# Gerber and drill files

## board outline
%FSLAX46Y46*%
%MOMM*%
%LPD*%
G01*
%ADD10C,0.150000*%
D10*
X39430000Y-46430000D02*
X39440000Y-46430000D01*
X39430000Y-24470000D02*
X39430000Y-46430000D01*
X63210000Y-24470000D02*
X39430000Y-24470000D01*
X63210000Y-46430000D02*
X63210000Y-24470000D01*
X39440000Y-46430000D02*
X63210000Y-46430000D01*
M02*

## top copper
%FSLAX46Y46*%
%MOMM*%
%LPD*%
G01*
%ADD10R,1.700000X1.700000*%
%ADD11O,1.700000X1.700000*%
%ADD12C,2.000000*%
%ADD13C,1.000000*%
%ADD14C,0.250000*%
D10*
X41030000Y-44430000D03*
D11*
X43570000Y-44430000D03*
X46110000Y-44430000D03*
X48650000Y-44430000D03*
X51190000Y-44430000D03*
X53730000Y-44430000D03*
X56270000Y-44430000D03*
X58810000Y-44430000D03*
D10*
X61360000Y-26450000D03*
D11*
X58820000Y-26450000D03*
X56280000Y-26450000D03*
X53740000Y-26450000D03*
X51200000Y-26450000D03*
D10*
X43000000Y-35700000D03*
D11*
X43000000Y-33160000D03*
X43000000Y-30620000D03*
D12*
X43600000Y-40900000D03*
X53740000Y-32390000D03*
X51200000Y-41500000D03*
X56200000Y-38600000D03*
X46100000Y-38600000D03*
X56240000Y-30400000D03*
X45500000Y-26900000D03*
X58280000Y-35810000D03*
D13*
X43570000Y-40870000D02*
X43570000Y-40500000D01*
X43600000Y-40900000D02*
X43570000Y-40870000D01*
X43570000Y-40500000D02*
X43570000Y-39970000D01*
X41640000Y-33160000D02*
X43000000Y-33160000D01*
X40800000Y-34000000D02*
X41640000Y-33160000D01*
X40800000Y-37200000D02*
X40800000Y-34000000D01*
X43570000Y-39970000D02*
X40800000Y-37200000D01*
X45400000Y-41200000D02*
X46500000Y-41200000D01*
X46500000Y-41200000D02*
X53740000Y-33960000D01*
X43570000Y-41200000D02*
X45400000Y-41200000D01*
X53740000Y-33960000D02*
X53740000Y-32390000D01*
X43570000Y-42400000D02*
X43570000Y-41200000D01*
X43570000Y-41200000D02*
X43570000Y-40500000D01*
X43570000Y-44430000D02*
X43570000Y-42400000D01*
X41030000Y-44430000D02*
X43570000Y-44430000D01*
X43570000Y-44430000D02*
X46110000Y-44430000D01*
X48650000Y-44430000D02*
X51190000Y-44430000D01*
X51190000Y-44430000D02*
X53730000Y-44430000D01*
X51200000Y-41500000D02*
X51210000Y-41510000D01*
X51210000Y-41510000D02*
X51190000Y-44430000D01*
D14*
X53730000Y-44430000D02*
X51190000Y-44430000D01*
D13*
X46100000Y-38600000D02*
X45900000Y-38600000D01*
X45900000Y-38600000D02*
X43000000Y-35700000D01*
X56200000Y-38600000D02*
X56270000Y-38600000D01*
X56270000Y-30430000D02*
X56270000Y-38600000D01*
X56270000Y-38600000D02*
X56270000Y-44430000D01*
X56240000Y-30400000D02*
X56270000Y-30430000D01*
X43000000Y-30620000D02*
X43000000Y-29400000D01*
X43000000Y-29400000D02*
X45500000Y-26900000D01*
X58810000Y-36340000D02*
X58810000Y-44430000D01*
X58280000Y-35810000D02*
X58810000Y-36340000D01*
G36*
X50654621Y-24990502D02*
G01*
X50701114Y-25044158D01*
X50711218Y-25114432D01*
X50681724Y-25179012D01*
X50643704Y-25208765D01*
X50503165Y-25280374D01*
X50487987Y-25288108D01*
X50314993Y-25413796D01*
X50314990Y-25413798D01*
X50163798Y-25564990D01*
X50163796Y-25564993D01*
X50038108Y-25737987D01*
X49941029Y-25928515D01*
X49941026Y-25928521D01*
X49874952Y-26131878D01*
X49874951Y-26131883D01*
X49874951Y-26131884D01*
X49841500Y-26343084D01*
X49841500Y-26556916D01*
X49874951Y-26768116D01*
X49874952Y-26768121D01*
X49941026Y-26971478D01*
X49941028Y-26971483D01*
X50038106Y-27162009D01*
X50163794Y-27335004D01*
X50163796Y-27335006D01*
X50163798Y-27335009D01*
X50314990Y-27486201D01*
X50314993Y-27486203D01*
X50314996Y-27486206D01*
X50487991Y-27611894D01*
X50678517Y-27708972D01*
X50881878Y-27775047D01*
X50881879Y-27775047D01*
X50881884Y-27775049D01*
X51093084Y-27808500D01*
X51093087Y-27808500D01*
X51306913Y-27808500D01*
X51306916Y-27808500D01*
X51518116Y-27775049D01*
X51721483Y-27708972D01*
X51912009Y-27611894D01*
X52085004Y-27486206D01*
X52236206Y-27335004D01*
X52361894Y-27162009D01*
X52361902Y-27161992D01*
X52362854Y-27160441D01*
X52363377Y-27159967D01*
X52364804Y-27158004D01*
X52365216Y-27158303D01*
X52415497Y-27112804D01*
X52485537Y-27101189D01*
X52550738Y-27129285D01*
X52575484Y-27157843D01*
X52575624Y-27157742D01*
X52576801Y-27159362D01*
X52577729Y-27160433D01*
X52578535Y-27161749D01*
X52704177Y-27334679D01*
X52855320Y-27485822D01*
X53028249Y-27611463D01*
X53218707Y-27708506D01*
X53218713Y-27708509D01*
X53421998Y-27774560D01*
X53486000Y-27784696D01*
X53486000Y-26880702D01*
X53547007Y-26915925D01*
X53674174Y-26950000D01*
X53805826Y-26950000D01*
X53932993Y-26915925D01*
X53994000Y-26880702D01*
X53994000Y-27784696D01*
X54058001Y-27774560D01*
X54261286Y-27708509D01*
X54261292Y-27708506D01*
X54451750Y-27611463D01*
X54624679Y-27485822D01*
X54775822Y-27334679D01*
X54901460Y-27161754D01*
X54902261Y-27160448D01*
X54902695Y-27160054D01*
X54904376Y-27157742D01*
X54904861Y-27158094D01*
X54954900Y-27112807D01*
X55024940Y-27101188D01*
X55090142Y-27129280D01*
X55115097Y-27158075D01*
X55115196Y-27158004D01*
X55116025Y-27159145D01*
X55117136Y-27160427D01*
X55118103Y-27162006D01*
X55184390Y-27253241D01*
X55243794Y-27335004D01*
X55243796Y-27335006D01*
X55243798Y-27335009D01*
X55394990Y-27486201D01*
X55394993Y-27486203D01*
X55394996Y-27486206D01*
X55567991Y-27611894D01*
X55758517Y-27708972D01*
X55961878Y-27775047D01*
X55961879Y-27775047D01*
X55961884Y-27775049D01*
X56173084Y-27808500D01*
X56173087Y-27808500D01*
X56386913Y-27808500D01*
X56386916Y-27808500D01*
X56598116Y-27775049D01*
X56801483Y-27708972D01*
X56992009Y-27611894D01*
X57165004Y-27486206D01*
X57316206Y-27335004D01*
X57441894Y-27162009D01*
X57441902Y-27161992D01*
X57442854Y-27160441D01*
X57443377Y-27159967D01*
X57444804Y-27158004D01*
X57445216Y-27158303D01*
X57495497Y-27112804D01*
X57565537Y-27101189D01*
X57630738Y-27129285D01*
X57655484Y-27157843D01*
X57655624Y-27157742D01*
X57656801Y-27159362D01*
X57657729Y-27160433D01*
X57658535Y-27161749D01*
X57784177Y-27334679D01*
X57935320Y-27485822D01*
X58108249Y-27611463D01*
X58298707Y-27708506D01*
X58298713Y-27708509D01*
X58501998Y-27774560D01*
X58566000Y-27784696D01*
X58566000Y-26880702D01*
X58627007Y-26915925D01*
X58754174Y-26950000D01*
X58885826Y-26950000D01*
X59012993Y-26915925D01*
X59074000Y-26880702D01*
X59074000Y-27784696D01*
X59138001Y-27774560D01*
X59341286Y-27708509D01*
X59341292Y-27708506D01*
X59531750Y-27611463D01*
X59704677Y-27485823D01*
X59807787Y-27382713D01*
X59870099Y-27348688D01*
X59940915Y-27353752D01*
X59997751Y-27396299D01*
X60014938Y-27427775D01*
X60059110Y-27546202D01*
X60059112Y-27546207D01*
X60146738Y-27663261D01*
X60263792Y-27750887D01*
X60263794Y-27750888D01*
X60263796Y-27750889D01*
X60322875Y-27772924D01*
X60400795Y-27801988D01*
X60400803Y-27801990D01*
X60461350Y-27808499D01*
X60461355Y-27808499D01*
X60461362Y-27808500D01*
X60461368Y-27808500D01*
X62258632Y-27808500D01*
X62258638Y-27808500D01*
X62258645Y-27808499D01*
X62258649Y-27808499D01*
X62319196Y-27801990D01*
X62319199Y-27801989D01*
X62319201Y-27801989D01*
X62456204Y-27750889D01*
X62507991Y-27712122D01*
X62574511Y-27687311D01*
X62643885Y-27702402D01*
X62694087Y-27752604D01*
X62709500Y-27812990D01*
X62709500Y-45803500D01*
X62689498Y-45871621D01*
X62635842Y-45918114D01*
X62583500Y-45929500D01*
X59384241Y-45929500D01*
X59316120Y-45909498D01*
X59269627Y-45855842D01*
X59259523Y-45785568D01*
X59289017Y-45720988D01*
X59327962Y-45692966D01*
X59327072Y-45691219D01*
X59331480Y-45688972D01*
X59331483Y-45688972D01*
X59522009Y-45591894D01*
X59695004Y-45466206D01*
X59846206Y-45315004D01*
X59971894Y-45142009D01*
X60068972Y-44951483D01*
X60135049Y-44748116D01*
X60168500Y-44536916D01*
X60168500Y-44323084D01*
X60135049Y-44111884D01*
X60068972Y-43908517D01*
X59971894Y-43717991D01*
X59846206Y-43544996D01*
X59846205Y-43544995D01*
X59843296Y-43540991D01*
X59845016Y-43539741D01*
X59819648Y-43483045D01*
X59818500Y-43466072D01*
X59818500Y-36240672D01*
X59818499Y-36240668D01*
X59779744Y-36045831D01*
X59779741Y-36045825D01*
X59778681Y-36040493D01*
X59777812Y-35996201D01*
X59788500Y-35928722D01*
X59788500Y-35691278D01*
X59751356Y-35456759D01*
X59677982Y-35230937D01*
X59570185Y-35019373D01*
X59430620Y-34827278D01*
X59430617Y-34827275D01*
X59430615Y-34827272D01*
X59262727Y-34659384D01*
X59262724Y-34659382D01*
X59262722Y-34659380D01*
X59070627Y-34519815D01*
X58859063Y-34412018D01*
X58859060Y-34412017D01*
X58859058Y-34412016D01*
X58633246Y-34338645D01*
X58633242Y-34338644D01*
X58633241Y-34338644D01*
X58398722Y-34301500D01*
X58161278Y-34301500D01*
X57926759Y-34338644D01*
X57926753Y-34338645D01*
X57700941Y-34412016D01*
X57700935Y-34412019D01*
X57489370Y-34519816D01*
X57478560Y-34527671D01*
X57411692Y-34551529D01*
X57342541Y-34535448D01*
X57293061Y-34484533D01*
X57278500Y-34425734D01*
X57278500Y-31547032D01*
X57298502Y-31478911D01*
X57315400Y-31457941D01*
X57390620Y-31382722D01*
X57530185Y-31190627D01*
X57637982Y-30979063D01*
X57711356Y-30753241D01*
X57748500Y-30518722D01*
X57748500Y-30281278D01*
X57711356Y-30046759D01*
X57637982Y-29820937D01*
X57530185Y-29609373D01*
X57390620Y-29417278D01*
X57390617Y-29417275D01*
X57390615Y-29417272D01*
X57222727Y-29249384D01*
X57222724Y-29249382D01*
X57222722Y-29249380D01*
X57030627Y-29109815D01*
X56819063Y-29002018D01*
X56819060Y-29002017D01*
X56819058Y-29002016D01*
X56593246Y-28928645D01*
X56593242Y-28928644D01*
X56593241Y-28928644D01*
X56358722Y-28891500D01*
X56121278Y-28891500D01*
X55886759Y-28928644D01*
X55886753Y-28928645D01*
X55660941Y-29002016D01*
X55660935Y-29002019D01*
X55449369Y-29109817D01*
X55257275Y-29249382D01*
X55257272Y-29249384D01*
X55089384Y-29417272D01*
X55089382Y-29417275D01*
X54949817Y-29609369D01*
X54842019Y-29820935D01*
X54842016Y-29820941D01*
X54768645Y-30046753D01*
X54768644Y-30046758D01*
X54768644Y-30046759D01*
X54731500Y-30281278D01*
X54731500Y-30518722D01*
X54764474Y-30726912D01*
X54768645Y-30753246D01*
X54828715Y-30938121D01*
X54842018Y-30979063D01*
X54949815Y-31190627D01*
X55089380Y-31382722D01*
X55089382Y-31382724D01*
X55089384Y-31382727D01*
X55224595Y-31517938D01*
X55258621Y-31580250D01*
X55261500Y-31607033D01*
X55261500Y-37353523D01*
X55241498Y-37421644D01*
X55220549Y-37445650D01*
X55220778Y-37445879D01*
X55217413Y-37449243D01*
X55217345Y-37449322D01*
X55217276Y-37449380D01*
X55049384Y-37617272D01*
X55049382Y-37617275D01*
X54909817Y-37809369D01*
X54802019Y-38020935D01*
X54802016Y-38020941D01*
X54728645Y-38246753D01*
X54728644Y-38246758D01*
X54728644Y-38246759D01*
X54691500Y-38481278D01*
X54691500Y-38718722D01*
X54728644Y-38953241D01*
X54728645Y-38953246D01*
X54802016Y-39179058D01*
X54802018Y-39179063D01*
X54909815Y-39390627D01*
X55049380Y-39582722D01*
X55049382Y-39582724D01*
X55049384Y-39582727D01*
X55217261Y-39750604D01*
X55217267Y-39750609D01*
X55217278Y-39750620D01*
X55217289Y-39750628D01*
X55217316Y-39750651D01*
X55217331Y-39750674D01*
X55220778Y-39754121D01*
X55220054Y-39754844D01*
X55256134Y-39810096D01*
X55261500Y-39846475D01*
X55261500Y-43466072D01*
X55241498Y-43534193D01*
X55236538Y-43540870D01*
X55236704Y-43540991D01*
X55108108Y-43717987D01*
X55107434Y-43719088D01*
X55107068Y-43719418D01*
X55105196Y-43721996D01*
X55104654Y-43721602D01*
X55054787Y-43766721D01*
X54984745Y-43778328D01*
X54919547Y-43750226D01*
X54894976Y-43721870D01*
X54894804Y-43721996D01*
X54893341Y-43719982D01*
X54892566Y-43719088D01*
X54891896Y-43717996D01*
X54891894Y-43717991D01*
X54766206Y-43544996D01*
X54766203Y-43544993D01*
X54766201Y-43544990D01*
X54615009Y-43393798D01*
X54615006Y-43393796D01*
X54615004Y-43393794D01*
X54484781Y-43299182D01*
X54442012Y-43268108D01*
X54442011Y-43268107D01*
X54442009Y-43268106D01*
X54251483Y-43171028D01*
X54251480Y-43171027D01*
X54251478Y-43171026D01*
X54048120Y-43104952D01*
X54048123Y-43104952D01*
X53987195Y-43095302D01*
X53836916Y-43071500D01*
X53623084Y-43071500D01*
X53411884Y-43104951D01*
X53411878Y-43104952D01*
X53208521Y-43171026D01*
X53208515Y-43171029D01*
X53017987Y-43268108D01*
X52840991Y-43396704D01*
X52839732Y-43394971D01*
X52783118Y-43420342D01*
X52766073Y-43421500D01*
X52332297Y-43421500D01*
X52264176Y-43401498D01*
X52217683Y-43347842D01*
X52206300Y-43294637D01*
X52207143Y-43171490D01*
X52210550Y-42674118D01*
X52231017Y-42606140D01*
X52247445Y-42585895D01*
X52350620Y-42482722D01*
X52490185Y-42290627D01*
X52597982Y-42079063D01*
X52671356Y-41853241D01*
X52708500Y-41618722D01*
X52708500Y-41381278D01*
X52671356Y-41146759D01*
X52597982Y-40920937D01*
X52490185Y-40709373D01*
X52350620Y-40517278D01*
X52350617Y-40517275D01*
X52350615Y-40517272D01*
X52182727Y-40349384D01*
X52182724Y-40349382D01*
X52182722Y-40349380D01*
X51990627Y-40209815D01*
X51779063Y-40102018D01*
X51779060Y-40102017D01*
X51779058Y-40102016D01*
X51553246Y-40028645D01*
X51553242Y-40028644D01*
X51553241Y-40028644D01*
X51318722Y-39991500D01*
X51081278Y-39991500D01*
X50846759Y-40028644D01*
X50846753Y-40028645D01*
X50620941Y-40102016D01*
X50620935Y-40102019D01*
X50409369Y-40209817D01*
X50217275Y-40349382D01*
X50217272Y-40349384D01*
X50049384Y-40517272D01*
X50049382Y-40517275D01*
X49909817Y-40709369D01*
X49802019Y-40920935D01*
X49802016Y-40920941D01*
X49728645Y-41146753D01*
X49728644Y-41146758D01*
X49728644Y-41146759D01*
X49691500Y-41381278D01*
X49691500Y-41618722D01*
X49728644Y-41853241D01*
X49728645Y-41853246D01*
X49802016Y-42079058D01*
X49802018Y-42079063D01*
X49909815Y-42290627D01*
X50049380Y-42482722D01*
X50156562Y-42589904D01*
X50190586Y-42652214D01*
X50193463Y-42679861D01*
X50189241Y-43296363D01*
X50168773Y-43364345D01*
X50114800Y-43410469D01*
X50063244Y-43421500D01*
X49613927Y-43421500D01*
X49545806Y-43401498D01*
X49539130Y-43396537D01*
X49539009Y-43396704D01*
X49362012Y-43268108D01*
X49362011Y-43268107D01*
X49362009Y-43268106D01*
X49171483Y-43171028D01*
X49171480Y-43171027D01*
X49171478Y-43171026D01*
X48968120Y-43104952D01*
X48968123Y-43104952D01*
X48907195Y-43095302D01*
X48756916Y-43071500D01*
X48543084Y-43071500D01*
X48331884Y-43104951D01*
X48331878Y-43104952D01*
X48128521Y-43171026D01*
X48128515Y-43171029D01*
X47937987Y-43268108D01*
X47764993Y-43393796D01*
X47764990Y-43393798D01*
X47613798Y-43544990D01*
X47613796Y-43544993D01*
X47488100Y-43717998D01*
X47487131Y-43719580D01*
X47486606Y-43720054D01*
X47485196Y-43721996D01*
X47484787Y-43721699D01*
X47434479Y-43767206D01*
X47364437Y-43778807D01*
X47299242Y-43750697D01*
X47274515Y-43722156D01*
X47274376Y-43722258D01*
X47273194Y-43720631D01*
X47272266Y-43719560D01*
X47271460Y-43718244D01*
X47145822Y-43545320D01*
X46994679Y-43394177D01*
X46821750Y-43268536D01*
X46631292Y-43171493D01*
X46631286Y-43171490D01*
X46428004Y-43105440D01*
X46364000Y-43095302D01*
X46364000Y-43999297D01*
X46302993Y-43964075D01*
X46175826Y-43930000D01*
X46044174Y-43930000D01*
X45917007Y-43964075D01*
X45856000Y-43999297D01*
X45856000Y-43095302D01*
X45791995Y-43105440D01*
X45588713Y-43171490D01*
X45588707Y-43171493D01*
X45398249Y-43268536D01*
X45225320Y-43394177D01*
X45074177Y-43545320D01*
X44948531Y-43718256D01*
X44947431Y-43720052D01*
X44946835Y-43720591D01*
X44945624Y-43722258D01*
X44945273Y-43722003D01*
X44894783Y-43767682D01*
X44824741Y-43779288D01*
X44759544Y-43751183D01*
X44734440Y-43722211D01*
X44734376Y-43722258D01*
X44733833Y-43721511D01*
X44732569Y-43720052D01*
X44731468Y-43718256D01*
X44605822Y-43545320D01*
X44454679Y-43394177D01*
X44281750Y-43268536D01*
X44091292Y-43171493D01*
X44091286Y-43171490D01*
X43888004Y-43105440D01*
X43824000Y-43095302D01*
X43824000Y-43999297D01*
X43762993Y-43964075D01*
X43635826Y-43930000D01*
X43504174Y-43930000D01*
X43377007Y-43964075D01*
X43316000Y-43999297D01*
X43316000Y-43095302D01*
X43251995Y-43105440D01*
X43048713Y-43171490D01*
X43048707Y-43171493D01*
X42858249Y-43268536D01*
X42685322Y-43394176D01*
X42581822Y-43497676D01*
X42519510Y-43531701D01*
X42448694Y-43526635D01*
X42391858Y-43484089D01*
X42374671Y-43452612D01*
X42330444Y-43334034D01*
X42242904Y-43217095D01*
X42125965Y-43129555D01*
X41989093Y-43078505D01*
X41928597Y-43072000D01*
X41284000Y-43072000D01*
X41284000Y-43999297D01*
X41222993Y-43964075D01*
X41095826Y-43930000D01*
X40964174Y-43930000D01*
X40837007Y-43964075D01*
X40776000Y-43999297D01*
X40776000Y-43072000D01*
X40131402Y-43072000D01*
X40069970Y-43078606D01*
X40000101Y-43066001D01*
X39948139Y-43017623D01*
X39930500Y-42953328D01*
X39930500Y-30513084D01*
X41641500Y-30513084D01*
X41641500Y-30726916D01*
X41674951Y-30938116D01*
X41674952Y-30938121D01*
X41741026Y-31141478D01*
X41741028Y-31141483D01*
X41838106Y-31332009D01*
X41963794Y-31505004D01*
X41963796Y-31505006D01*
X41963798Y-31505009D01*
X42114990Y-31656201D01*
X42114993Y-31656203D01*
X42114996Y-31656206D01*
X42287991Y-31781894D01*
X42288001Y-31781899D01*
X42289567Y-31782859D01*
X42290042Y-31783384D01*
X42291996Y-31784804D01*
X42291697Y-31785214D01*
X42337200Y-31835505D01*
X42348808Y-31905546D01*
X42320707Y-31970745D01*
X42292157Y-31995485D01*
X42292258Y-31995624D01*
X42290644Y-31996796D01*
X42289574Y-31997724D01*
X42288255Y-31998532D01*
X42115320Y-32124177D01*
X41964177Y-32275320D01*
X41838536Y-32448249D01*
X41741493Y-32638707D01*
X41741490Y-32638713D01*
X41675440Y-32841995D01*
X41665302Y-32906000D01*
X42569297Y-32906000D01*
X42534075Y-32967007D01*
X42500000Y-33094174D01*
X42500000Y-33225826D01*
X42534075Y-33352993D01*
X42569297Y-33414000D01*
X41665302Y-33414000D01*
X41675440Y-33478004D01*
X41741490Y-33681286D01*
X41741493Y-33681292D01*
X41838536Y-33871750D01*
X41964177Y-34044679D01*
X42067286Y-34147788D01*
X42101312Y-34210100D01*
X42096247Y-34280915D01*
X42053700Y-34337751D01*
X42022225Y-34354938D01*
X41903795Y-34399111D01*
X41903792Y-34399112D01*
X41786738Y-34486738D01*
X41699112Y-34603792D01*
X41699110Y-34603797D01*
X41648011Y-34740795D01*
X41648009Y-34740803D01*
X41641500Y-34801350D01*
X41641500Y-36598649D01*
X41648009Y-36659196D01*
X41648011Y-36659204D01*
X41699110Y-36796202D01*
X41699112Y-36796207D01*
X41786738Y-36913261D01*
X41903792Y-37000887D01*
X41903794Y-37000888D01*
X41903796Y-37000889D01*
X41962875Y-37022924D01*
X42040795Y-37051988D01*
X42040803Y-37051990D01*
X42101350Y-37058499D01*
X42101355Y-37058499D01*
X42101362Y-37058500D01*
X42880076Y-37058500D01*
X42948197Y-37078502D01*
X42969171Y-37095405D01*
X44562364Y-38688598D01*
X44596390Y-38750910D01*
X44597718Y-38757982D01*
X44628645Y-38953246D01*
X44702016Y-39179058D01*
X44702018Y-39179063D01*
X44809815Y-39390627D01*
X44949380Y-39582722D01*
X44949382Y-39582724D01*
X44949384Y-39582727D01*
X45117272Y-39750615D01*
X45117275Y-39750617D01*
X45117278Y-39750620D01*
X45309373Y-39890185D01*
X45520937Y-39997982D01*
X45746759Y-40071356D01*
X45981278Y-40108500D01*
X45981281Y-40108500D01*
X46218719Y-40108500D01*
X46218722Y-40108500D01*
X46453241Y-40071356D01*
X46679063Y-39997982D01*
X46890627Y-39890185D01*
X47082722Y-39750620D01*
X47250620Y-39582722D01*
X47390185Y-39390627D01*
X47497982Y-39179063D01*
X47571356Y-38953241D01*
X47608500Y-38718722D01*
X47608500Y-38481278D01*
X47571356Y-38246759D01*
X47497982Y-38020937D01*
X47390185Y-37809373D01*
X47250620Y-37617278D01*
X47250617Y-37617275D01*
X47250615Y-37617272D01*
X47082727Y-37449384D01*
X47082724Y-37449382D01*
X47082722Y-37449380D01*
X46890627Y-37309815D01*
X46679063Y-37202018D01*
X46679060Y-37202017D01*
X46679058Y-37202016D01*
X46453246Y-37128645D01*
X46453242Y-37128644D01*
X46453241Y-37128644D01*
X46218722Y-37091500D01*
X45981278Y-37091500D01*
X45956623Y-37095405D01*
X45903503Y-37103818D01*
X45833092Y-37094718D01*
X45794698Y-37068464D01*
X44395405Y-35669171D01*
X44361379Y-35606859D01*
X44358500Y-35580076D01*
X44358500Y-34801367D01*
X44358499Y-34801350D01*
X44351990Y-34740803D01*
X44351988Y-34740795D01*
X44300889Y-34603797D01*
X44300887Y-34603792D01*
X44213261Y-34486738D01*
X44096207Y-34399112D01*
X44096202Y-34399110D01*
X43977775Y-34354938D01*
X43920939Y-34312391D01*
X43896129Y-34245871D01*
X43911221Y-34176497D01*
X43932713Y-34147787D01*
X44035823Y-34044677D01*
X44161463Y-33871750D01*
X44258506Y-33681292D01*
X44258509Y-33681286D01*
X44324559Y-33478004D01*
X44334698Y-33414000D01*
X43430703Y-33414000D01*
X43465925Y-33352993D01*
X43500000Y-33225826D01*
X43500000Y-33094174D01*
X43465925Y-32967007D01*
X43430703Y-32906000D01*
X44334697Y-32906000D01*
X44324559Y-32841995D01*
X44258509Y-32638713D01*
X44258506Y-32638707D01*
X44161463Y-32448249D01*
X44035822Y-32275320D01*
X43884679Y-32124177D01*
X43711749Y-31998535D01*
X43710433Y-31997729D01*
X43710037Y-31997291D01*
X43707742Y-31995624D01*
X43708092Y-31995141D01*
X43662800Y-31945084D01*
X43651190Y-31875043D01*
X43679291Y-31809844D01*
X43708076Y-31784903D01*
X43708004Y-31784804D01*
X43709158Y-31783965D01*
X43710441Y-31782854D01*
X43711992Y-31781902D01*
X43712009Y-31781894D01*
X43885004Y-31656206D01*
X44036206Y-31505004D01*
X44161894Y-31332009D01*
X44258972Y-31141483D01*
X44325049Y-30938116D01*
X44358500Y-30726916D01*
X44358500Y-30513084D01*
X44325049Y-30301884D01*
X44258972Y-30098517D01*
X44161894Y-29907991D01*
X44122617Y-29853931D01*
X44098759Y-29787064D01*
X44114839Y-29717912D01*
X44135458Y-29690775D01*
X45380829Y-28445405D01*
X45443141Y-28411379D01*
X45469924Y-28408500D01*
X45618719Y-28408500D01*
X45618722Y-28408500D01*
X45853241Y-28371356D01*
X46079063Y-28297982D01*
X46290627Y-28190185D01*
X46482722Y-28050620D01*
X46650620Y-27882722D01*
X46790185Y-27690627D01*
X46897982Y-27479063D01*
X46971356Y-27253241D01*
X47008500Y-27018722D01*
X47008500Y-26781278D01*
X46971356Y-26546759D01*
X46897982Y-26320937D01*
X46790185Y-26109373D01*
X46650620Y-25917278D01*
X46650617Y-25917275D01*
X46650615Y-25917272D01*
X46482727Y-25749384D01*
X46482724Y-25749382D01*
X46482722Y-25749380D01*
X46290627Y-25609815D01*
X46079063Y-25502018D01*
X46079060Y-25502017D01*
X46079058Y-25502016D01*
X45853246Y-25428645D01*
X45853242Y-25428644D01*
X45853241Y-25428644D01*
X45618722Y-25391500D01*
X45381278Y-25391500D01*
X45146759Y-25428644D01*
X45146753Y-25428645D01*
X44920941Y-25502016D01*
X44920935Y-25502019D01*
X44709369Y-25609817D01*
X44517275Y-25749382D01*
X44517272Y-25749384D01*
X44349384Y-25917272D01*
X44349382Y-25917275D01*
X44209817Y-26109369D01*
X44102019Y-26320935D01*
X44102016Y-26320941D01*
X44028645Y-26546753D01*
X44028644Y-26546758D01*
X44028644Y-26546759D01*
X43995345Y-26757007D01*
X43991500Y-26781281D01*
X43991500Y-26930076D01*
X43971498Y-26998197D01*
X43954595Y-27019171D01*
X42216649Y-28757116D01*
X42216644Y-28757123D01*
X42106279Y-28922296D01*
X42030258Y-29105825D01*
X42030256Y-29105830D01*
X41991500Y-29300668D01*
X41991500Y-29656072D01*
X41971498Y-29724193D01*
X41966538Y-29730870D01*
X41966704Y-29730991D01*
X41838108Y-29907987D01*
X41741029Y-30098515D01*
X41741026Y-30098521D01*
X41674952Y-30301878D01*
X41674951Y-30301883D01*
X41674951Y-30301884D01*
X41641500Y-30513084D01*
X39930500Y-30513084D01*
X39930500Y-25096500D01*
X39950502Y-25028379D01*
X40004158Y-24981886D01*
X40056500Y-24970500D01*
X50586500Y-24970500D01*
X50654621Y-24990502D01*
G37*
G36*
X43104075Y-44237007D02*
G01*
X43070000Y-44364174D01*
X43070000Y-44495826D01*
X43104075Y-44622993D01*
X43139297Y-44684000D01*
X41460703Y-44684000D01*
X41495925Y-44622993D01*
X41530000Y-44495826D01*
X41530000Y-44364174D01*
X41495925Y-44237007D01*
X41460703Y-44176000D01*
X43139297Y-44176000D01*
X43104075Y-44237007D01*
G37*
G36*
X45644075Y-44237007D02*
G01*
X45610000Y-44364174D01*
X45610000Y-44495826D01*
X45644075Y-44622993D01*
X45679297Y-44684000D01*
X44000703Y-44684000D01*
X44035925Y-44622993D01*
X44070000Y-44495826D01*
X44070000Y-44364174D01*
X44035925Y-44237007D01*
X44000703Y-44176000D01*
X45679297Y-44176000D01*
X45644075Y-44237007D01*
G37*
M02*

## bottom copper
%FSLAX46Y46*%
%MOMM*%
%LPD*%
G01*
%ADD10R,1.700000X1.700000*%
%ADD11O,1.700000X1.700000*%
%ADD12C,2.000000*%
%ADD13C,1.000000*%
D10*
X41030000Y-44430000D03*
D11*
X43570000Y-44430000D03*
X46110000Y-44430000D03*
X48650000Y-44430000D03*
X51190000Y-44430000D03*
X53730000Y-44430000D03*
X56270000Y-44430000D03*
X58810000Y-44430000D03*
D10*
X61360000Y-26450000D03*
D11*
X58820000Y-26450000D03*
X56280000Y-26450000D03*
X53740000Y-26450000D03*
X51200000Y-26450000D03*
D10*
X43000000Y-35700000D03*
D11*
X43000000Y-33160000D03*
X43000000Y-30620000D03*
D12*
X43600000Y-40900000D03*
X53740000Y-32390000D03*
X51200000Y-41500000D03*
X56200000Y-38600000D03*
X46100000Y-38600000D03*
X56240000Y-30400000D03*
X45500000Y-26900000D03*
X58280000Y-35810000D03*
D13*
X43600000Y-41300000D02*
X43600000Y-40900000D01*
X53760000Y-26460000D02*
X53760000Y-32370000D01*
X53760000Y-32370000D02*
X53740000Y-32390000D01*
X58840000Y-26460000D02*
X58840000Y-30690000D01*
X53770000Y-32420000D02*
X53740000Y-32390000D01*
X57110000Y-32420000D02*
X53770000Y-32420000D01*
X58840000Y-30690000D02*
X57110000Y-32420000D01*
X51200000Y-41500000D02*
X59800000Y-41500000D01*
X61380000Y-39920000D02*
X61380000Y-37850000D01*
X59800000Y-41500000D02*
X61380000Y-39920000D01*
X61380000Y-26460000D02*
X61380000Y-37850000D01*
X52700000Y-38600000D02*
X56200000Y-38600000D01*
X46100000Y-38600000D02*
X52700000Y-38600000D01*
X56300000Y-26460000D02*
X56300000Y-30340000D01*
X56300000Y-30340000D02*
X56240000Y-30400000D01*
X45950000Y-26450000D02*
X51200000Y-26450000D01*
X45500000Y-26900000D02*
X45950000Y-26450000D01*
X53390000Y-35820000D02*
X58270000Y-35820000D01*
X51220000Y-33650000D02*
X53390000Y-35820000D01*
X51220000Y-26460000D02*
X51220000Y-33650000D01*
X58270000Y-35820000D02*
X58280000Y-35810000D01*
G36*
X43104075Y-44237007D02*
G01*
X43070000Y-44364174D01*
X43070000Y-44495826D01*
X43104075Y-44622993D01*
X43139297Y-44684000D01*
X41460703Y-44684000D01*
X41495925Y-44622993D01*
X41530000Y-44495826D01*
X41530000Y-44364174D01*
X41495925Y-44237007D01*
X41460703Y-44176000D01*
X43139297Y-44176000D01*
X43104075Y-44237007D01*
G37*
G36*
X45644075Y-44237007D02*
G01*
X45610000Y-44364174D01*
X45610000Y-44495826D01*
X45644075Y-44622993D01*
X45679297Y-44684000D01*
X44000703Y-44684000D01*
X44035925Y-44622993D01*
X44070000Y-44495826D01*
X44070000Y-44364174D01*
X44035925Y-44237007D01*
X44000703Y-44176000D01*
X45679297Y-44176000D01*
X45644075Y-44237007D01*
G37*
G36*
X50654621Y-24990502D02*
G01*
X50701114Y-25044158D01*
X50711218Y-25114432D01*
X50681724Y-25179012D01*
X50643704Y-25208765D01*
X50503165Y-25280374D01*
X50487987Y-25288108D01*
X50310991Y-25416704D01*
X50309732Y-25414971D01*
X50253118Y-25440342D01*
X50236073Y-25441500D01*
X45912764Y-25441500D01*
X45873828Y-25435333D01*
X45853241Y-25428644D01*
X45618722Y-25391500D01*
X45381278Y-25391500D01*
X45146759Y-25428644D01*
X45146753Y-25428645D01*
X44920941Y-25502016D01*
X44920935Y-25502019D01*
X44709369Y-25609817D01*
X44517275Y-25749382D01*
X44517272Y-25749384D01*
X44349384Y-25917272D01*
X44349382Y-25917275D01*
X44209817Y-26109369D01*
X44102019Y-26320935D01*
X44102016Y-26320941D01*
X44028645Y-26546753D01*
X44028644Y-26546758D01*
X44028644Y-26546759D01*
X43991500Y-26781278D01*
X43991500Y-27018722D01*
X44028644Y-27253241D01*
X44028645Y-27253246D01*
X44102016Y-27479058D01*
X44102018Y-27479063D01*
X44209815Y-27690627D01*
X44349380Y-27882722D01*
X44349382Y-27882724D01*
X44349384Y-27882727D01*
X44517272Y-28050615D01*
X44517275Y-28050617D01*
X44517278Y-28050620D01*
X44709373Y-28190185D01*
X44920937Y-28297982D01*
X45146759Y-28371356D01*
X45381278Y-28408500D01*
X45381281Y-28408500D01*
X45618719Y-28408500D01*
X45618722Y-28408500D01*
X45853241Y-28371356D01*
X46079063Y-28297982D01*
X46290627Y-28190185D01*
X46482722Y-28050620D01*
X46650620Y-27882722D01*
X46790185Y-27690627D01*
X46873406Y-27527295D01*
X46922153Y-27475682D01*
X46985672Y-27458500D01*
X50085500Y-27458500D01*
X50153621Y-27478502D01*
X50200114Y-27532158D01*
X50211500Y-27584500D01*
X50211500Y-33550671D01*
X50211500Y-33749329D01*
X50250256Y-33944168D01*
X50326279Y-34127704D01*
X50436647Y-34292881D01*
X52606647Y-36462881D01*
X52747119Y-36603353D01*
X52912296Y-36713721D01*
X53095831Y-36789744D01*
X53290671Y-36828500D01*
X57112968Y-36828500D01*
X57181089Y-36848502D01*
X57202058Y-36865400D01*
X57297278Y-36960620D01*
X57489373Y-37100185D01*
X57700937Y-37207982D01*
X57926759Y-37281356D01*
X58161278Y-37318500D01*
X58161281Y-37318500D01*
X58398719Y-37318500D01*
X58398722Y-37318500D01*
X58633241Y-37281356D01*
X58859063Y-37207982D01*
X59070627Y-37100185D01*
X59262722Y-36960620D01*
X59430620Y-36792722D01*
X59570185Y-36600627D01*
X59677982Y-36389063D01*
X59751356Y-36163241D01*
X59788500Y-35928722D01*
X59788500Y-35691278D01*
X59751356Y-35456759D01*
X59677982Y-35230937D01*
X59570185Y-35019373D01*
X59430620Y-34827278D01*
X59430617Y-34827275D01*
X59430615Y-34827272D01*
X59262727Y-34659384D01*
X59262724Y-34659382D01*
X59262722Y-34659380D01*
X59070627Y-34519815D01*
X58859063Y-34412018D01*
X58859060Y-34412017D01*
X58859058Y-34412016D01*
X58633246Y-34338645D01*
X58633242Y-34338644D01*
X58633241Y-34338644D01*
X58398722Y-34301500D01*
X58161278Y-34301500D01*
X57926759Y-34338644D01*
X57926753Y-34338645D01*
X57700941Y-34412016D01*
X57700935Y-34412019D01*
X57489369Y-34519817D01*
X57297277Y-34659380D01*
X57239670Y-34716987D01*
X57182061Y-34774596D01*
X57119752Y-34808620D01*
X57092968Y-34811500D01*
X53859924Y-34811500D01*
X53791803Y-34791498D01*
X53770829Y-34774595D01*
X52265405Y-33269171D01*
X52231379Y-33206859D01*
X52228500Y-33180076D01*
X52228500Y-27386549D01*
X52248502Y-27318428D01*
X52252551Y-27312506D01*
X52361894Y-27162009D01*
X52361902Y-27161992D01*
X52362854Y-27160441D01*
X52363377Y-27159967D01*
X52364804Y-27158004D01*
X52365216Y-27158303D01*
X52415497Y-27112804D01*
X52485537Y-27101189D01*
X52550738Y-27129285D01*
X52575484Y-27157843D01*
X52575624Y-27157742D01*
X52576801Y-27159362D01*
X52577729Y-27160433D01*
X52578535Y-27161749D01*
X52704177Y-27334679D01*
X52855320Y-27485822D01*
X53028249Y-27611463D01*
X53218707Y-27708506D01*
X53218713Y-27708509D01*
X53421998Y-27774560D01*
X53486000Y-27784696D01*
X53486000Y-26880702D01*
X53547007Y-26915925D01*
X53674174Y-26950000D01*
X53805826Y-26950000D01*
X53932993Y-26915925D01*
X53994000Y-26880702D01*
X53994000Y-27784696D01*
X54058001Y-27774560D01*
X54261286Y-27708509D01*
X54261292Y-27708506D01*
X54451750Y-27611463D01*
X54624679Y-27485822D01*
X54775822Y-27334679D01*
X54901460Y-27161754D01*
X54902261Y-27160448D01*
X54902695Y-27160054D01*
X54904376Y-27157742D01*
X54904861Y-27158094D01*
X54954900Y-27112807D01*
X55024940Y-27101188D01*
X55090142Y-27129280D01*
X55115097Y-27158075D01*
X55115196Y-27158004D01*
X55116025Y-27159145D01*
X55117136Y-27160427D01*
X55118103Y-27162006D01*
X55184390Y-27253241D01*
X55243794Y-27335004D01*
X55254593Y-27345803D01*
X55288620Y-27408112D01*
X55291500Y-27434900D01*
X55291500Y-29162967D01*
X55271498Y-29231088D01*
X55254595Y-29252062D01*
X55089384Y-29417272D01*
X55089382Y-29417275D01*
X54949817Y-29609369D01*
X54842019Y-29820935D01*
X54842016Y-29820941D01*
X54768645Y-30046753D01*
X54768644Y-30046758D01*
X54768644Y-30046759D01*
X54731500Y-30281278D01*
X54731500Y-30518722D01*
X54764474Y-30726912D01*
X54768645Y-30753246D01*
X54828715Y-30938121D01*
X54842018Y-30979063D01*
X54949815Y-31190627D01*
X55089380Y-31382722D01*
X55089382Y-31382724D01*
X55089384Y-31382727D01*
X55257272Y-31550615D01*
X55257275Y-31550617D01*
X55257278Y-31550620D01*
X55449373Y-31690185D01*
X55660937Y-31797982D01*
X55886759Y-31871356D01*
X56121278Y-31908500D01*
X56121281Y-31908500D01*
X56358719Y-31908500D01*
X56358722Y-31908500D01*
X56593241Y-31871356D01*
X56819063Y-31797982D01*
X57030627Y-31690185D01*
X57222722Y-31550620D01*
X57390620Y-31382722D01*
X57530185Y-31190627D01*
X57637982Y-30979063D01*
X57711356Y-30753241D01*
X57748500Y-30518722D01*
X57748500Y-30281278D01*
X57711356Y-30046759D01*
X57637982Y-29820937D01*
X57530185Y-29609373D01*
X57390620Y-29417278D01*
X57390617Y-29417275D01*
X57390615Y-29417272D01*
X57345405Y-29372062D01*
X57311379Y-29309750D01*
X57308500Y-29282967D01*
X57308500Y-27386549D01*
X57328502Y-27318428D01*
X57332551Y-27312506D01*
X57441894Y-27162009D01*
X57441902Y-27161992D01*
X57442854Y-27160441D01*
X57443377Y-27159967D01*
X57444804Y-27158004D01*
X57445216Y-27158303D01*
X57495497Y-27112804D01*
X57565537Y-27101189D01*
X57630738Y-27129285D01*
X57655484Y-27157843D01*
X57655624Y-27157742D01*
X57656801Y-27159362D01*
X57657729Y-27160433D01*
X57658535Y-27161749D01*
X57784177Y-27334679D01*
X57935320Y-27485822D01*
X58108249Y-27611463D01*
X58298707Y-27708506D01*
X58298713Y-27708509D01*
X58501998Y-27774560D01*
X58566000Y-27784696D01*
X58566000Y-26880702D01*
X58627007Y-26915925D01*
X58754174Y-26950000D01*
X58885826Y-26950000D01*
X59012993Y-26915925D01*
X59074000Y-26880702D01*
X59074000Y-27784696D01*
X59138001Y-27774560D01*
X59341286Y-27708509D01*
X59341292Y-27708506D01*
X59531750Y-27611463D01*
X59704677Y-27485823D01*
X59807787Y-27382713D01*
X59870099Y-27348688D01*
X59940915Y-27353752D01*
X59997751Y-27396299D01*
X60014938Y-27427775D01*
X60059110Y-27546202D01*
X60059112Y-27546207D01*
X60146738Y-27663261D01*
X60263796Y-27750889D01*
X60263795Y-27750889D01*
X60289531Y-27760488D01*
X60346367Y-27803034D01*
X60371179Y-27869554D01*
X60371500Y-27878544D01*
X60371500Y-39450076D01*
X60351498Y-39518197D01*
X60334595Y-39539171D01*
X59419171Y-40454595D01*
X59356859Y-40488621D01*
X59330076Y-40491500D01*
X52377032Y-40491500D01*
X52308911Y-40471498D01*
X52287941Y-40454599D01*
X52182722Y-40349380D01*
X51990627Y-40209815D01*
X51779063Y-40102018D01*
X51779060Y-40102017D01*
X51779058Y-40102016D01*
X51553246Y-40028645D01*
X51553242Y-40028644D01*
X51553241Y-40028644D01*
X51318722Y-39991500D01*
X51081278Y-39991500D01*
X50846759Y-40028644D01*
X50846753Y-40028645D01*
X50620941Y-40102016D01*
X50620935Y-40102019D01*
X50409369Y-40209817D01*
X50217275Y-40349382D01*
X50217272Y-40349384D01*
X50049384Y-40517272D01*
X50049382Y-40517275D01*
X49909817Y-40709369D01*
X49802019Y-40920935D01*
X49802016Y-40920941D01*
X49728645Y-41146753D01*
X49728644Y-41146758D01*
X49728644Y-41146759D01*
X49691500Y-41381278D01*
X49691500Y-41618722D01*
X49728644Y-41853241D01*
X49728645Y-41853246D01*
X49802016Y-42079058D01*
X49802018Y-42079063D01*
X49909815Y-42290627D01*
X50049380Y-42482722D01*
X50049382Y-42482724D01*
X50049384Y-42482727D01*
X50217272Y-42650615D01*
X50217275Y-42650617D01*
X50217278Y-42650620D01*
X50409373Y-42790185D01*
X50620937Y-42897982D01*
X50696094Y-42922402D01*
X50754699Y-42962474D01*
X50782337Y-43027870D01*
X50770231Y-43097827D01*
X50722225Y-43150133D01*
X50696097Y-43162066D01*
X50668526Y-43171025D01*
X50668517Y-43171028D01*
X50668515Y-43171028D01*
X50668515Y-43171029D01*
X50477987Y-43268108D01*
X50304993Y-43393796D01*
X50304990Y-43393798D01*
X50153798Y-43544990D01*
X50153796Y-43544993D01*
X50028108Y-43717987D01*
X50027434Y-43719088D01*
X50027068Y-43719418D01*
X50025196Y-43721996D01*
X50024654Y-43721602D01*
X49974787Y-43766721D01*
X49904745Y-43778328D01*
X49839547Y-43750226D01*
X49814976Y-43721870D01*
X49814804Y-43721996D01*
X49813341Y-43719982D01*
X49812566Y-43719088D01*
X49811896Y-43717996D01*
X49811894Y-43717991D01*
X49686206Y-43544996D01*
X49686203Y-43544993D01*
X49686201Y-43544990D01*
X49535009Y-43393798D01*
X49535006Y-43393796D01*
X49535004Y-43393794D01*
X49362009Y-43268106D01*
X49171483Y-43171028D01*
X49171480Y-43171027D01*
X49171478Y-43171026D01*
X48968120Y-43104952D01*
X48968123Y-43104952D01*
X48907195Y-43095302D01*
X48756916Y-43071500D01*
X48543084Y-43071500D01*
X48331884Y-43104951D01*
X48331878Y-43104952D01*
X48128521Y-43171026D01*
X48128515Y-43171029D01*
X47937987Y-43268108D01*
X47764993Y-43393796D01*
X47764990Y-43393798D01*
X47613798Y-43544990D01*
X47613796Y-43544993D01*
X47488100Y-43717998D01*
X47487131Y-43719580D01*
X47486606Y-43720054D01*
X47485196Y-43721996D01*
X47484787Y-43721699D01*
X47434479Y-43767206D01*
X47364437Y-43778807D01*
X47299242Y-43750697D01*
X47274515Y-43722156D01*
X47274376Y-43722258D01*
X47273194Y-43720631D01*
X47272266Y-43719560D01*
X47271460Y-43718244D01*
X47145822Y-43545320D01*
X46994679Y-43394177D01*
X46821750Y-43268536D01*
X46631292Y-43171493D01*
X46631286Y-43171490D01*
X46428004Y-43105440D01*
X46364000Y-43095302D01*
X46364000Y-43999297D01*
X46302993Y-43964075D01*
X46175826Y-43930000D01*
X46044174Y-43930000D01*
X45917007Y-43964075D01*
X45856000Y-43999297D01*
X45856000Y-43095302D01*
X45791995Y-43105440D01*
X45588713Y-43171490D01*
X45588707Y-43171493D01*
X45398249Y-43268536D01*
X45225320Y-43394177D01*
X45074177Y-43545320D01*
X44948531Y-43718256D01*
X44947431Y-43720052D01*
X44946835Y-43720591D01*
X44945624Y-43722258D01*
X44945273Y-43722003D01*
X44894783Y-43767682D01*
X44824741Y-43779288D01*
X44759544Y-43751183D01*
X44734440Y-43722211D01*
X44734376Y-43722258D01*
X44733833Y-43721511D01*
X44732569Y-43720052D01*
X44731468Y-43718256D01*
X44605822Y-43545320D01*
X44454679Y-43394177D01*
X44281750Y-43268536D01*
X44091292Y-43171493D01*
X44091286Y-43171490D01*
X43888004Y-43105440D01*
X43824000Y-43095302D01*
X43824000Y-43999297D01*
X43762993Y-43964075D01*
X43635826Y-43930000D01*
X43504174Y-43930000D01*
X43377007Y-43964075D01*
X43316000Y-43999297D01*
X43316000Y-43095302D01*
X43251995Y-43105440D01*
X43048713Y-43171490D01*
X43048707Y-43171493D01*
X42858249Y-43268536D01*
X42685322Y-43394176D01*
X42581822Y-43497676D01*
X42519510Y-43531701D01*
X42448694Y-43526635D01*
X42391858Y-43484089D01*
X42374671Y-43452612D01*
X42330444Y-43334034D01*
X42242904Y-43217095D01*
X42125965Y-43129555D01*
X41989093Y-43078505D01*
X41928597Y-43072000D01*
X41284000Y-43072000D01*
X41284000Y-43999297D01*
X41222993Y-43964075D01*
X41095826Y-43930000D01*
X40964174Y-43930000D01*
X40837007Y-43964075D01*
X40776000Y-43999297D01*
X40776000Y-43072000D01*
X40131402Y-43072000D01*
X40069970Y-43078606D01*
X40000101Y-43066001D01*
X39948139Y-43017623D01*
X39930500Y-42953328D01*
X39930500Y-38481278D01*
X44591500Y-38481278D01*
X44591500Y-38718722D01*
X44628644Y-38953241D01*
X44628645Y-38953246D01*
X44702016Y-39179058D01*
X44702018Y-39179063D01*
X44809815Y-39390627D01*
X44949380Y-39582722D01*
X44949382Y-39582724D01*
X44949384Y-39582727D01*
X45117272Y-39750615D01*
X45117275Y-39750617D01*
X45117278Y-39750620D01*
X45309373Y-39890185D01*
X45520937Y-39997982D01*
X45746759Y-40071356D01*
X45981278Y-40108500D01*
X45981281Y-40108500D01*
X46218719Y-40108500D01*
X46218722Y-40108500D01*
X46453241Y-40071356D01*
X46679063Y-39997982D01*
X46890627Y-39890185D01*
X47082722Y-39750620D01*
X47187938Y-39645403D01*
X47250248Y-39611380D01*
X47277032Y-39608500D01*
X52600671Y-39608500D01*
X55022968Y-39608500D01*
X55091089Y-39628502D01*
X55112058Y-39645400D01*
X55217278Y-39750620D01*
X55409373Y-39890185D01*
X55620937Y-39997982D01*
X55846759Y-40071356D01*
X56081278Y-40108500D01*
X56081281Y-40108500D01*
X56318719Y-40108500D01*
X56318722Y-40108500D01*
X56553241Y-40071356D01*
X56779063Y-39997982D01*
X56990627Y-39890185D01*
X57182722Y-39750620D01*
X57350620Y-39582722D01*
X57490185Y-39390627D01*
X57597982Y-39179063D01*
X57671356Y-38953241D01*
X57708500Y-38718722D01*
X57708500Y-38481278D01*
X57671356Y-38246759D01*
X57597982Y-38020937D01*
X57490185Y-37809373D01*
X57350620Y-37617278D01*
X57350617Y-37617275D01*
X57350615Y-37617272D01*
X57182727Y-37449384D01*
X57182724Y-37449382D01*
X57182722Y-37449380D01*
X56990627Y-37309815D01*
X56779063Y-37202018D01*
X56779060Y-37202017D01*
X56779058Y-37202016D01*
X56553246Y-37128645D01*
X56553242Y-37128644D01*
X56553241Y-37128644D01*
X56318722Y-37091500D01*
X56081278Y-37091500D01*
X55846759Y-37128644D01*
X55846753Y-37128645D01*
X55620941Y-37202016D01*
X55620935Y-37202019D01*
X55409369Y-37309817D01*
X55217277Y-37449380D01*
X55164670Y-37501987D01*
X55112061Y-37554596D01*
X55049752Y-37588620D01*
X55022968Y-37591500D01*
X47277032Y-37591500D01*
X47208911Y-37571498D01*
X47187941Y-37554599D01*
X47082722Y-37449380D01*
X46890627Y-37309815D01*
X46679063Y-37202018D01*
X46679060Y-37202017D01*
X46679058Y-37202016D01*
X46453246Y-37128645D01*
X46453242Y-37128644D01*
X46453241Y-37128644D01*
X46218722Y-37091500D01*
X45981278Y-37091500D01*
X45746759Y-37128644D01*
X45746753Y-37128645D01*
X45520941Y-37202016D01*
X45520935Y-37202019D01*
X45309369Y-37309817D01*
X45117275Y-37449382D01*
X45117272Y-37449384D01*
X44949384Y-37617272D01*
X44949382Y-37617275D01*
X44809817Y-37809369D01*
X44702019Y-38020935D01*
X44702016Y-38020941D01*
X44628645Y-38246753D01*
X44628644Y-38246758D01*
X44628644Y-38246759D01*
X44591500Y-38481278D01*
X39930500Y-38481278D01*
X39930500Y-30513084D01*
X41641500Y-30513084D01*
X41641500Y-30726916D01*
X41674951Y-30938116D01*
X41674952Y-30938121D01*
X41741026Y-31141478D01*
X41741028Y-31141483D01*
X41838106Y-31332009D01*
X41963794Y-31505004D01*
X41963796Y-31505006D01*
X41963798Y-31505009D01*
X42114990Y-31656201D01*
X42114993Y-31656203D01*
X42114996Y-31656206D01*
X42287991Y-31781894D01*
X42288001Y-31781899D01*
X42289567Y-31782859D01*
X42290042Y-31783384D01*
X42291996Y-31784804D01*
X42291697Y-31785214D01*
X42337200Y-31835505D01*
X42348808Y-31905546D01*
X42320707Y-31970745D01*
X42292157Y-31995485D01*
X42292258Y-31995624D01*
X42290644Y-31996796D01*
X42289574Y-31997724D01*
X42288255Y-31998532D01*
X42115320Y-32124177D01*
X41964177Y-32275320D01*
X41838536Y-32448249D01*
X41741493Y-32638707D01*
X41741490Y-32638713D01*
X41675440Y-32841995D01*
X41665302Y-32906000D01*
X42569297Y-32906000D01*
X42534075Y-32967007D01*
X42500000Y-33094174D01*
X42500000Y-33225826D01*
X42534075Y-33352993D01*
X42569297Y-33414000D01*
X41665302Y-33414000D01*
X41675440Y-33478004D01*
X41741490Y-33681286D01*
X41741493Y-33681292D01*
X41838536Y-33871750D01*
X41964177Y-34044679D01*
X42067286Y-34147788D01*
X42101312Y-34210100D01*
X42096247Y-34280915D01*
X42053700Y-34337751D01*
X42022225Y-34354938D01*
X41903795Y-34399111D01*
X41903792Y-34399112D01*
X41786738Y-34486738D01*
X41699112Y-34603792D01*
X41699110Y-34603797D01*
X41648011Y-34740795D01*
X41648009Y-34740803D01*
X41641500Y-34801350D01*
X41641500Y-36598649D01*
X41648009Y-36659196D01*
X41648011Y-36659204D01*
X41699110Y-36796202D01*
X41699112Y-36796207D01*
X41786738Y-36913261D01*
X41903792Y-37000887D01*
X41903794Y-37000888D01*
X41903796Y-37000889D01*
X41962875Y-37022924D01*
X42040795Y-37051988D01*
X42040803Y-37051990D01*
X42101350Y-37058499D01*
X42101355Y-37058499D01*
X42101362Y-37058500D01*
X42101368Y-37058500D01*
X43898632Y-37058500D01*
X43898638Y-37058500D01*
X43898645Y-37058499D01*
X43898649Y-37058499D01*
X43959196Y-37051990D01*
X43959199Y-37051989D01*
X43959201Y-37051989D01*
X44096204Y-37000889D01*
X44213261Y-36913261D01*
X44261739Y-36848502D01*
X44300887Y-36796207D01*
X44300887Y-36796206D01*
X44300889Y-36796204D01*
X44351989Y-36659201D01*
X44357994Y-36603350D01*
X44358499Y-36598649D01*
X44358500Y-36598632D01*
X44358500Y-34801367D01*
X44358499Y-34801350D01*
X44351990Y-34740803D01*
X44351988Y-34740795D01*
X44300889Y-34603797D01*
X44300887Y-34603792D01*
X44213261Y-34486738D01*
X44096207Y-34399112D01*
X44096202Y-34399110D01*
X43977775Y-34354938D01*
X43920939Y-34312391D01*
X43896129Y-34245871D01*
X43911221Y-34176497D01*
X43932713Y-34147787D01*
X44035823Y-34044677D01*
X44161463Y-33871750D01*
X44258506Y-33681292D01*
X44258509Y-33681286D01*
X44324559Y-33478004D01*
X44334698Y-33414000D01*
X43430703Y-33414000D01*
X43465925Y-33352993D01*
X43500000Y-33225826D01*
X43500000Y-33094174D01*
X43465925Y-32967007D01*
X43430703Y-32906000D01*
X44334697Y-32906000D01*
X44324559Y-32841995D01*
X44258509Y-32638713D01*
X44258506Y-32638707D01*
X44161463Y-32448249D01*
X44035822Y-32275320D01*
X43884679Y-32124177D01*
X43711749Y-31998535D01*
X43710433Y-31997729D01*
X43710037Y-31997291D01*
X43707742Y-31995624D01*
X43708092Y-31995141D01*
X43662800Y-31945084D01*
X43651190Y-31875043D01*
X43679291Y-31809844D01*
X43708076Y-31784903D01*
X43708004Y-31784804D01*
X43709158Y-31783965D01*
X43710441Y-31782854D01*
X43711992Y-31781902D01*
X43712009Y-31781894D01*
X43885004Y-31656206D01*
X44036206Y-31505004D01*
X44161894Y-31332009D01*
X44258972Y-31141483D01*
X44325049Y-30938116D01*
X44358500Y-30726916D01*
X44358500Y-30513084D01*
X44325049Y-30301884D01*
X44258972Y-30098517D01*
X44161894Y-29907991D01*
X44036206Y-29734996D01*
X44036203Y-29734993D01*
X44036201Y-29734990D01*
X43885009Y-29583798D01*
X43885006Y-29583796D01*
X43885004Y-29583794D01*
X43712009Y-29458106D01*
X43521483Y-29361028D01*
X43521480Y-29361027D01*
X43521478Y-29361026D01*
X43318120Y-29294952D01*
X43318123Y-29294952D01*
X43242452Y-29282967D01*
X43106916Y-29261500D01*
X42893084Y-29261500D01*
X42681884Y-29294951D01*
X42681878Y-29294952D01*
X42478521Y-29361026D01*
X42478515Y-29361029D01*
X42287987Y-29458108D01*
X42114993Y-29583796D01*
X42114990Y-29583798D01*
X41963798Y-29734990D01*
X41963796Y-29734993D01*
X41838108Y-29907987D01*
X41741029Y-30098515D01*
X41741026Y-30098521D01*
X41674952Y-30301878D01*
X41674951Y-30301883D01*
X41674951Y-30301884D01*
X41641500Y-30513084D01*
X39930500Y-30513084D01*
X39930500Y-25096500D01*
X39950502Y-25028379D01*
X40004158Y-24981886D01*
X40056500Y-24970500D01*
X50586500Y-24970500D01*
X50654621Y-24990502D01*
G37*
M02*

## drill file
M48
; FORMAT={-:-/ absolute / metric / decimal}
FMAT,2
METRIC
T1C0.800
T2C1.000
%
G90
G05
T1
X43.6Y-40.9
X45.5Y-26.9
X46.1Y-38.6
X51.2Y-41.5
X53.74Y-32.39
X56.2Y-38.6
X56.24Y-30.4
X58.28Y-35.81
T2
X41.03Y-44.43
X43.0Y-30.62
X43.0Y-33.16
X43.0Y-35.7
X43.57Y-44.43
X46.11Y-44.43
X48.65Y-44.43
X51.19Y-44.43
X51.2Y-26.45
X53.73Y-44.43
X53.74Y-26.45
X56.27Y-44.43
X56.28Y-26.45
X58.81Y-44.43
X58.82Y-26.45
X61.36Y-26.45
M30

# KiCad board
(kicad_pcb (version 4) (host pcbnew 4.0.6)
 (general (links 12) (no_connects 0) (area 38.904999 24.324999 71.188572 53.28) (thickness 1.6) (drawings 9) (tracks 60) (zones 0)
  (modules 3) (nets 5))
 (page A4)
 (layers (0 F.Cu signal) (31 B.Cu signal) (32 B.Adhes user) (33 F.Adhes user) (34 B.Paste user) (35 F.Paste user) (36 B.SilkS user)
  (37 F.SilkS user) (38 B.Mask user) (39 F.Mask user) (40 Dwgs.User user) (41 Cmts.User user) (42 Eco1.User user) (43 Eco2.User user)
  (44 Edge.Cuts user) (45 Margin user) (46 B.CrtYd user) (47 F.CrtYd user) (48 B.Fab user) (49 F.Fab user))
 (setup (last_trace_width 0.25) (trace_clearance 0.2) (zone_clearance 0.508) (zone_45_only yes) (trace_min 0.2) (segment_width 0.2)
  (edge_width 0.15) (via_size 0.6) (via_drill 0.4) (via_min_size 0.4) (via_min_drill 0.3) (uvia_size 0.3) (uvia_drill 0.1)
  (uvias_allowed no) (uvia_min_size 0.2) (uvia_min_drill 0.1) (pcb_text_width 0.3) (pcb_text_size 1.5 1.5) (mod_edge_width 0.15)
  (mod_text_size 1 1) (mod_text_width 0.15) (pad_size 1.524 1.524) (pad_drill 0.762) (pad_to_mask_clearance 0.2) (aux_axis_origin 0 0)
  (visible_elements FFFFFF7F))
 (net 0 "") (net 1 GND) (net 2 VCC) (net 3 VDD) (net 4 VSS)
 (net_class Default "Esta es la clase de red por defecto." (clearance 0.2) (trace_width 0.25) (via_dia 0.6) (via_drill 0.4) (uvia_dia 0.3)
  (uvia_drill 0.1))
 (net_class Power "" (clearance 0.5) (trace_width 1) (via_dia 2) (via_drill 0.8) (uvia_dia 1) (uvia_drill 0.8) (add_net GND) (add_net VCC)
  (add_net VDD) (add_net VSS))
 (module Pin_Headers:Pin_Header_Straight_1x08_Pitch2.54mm (layer B.Cu) (at 41.03 44.43 270)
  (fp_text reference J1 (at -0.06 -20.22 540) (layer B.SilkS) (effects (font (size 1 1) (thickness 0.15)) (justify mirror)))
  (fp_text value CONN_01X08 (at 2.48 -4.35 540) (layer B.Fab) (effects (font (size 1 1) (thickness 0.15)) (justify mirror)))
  (pad 1 thru_hole rect (at 0 0 270) (size 1.7 1.7) (drill 1) (layers *.Cu *.Mask) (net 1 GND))
  (pad 2 thru_hole oval (at 0 -2.54 270) (size 1.7 1.7) (drill 1) (layers *.Cu *.Mask) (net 1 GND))
  (pad 3 thru_hole oval (at 0 -5.08 270) (size 1.7 1.7) (drill 1) (layers *.Cu *.Mask) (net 1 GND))
  (pad 4 thru_hole oval (at 0 -7.62 270) (size 1.7 1.7) (drill 1) (layers *.Cu *.Mask) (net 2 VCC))
  (pad 5 thru_hole oval (at 0 -10.16 270) (size 1.7 1.7) (drill 1) (layers *.Cu *.Mask) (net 2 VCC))
  (pad 6 thru_hole oval (at 0 -12.7 270) (size 1.7 1.7) (drill 1) (layers *.Cu *.Mask) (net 2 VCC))
  (pad 7 thru_hole oval (at 0 -15.24 270) (size 1.7 1.7) (drill 1) (layers *.Cu *.Mask) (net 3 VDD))
  (pad 8 thru_hole oval (at 0 -17.78 270) (size 1.7 1.7) (drill 1) (layers *.Cu *.Mask) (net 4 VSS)))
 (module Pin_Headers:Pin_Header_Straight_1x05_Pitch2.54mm (layer F.Cu) (at 61.36 26.45 270)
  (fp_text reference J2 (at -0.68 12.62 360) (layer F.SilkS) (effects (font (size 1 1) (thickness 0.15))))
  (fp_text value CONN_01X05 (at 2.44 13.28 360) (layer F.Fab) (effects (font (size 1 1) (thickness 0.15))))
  (pad 1 thru_hole rect (at 0 0 270) (size 1.7 1.7) (drill 1) (layers *.Cu *.Mask) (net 2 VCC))
  (pad 2 thru_hole oval (at 0 2.54 270) (size 1.7 1.7) (drill 1) (layers *.Cu *.Mask) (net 1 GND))
  (pad 3 thru_hole oval (at 0 5.08 270) (size 1.7 1.7) (drill 1) (layers *.Cu *.Mask) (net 3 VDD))
  (pad 4 thru_hole oval (at 0 7.62 270) (size 1.7 1.7) (drill 1) (layers *.Cu *.Mask) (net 1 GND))
  (pad 5 thru_hole oval (at 0 10.16 270) (size 1.7 1.7) (drill 1) (layers *.Cu *.Mask) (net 4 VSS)))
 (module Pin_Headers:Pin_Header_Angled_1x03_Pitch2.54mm (layer B.Cu) (at 43 35.7)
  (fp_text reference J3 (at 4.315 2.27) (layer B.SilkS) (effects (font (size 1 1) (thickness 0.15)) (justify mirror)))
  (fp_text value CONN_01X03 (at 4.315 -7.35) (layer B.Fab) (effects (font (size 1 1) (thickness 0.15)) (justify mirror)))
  (pad 1 thru_hole rect (at 0 0) (size 1.7 1.7) (drill 1) (layers *.Cu *.Mask) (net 3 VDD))
  (pad 2 thru_hole oval (at 0 -2.54) (size 1.7 1.7) (drill 1) (layers *.Cu *.Mask) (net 1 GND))
  (pad 3 thru_hole oval (at 0 -5.08) (size 1.7 1.7) (drill 1) (layers *.Cu *.Mask) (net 4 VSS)))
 (gr_line (start 39.43 46.43) (end 39.44 46.43) (angle 90) (layer Edge.Cuts) (width 0.15))
 (gr_line (start 39.43 24.47) (end 39.43 46.43) (angle 90) (layer Edge.Cuts) (width 0.15))
 (gr_line (start 63.21 24.47) (end 39.43 24.47) (angle 90) (layer Edge.Cuts) (width 0.15))
 (gr_line (start 63.21 46.43) (end 63.21 24.47) (angle 90) (layer Edge.Cuts) (width 0.15))
 (gr_line (start 39.44 46.43) (end 63.21 46.43) (angle 90) (layer Edge.Cuts) (width 0.15))
 (segment (start 43.6 41.3) (end 43.6 40.9) (width 1) (layer B.Cu) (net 1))
 (segment (start 43.57 40.87) (end 43.57 40.5) (width 1) (layer F.Cu) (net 1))
 (segment (start 43.6 40.9) (end 43.57 40.87) (width 1) (layer F.Cu) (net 1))
 (via (at 43.6 40.9) (size 2) (drill 0.8) (layers F.Cu B.Cu) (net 1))
 (segment (start 43.57 40.5) (end 43.57 39.97) (width 1) (layer F.Cu) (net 1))
 (segment (start 41.64 33.16) (end 43 33.16) (width 1) (layer F.Cu) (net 1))
 (segment (start 40.8 34) (end 41.64 33.16) (width 1) (layer F.Cu) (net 1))
 (segment (start 40.8 37.2) (end 40.8 34) (width 1) (layer F.Cu) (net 1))
 (segment (start 43.57 39.97) (end 40.8 37.2) (width 1) (layer F.Cu) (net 1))
 (segment (start 45.4 41.2) (end 46.5 41.2) (width 1) (layer F.Cu) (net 1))
 (segment (start 46.5 41.2) (end 53.74 33.96) (width 1) (layer F.Cu) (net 1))
 (segment (start 43.57 41.2) (end 45.4 41.2) (width 1) (layer F.Cu) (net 1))
 (via (at 53.74 32.39) (size 2) (drill 0.8) (layers F.Cu B.Cu) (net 1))
 (segment (start 53.74 33.96) (end 53.74 32.39) (width 1) (layer F.Cu) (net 1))
 (segment (start 43.57 42.4) (end 43.57 41.2) (width 1) (layer F.Cu) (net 1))
 (segment (start 43.57 41.2) (end 43.57 40.5) (width 1) (layer F.Cu) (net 1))
 (segment (start 43.57 44.43) (end 43.57 42.4) (width 1) (layer F.Cu) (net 1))
 (segment (start 41.03 44.43) (end 43.57 44.43) (width 1) (layer F.Cu) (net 1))
 (segment (start 43.57 44.43) (end 46.11 44.43) (width 1) (layer F.Cu) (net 1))
 (segment (start 53.76 26.46) (end 53.76 32.37) (width 1) (layer B.Cu) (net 1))
 (segment (start 53.76 32.37) (end 53.74 32.39) (width 1) (layer B.Cu) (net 1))
 (segment (start 58.84 26.46) (end 58.84 30.69) (width 1) (layer B.Cu) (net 1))
 (segment (start 53.77 32.42) (end 53.74 32.39) (width 1) (layer B.Cu) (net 1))
 (segment (start 57.11 32.42) (end 53.77 32.42) (width 1) (layer B.Cu) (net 1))
 (segment (start 58.84 30.69) (end 57.11 32.42) (width 1) (layer B.Cu) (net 1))
 (segment (start 51.2 41.5) (end 59.8 41.5) (width 1) (layer B.Cu) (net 2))
 (segment (start 61.38 39.92) (end 61.38 37.85) (width 1) (layer B.Cu) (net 2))
 (segment (start 59.8 41.5) (end 61.38 39.92) (width 1) (layer B.Cu) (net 2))
 (segment (start 48.65 44.43) (end 51.19 44.43) (width 1) (layer F.Cu) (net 2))
 (segment (start 51.19 44.43) (end 53.73 44.43) (width 1) (layer F.Cu) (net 2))
 (segment (start 61.38 26.46) (end 61.38 37.85) (width 1) (layer B.Cu) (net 2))
 (via (at 51.2 41.5) (size 2) (drill 0.8) (layers F.Cu B.Cu) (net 2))
 (segment (start 51.2 41.5) (end 51.21 41.51) (width 1) (layer F.Cu) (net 2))
 (segment (start 51.21 41.51) (end 51.19 44.43) (width 1) (layer F.Cu) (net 2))
 (segment (start 53.73 44.43) (end 51.19 44.43) (width 0.25) (layer F.Cu) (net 2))
 (segment (start 46.1 38.6) (end 45.9 38.6) (width 1) (layer F.Cu) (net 3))
 (segment (start 45.9 38.6) (end 43 35.7) (width 1) (layer F.Cu) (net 3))
 (segment (start 56.2 38.6) (end 56.27 38.6) (width 1) (layer F.Cu) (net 3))
 (via (at 56.2 38.6) (size 2) (drill 0.8) (layers F.Cu B.Cu) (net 3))
 (segment (start 52.7 38.6) (end 56.2 38.6) (width 1) (layer B.Cu) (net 3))
 (segment (start 46.1 38.6) (end 52.7 38.6) (width 1) (layer B.Cu) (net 3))
 (via (at 46.1 38.6) (size 2) (drill 0.8) (layers F.Cu B.Cu) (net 3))
 (segment (start 56.3 26.46) (end 56.3 30.34) (width 1) (layer B.Cu) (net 3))
 (segment (start 56.27 30.43) (end 56.27 38.6) (width 1) (layer F.Cu) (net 3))
 (segment (start 56.27 38.6) (end 56.27 44.43) (width 1) (layer F.Cu) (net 3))
 (segment (start 56.24 30.4) (end 56.27 30.43) (width 1) (layer F.Cu) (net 3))
 (via (at 56.24 30.4) (size 2) (drill 0.8) (layers F.Cu B.Cu) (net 3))
 (segment (start 56.3 30.34) (end 56.24 30.4) (width 1) (layer B.Cu) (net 3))
 (segment (start 43 30.62) (end 43 29.4) (width 1) (layer F.Cu) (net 4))
 (segment (start 43 29.4) (end 45.5 26.9) (width 1) (layer F.Cu) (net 4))
 (segment (start 45.95 26.45) (end 51.2 26.45) (width 1) (layer B.Cu) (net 4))
 (segment (start 45.5 26.9) (end 45.95 26.45) (width 1) (layer B.Cu) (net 4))
 (via (at 45.5 26.9) (size 2) (drill 0.8) (layers F.Cu B.Cu) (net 4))
 (segment (start 53.39 35.82) (end 58.27 35.82) (width 1) (layer B.Cu) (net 4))
 (segment (start 51.22 33.65) (end 53.39 35.82) (width 1) (layer B.Cu) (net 4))
 (segment (start 51.22 26.46) (end 51.22 33.65) (width 1) (layer B.Cu) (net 4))
 (segment (start 58.81 36.34) (end 58.81 44.43) (width 1) (layer F.Cu) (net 4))
 (segment (start 58.28 35.81) (end 58.81 36.34) (width 1) (layer F.Cu) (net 4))
 (via (at 58.28 35.81) (size 2) (drill 0.8) (layers F.Cu B.Cu) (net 4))
 (segment (start 58.27 35.82) (end 58.28 35.81) (width 1) (layer B.Cu) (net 4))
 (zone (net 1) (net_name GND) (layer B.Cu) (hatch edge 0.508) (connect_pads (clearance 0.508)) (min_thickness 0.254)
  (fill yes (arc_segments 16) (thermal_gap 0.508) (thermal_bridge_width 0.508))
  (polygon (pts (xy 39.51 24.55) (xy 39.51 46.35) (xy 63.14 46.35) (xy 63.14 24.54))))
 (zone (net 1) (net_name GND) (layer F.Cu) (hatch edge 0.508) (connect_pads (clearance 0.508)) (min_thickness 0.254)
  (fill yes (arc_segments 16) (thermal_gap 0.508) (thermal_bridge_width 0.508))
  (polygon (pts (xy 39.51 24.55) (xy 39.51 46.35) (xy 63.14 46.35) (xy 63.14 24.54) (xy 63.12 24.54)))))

